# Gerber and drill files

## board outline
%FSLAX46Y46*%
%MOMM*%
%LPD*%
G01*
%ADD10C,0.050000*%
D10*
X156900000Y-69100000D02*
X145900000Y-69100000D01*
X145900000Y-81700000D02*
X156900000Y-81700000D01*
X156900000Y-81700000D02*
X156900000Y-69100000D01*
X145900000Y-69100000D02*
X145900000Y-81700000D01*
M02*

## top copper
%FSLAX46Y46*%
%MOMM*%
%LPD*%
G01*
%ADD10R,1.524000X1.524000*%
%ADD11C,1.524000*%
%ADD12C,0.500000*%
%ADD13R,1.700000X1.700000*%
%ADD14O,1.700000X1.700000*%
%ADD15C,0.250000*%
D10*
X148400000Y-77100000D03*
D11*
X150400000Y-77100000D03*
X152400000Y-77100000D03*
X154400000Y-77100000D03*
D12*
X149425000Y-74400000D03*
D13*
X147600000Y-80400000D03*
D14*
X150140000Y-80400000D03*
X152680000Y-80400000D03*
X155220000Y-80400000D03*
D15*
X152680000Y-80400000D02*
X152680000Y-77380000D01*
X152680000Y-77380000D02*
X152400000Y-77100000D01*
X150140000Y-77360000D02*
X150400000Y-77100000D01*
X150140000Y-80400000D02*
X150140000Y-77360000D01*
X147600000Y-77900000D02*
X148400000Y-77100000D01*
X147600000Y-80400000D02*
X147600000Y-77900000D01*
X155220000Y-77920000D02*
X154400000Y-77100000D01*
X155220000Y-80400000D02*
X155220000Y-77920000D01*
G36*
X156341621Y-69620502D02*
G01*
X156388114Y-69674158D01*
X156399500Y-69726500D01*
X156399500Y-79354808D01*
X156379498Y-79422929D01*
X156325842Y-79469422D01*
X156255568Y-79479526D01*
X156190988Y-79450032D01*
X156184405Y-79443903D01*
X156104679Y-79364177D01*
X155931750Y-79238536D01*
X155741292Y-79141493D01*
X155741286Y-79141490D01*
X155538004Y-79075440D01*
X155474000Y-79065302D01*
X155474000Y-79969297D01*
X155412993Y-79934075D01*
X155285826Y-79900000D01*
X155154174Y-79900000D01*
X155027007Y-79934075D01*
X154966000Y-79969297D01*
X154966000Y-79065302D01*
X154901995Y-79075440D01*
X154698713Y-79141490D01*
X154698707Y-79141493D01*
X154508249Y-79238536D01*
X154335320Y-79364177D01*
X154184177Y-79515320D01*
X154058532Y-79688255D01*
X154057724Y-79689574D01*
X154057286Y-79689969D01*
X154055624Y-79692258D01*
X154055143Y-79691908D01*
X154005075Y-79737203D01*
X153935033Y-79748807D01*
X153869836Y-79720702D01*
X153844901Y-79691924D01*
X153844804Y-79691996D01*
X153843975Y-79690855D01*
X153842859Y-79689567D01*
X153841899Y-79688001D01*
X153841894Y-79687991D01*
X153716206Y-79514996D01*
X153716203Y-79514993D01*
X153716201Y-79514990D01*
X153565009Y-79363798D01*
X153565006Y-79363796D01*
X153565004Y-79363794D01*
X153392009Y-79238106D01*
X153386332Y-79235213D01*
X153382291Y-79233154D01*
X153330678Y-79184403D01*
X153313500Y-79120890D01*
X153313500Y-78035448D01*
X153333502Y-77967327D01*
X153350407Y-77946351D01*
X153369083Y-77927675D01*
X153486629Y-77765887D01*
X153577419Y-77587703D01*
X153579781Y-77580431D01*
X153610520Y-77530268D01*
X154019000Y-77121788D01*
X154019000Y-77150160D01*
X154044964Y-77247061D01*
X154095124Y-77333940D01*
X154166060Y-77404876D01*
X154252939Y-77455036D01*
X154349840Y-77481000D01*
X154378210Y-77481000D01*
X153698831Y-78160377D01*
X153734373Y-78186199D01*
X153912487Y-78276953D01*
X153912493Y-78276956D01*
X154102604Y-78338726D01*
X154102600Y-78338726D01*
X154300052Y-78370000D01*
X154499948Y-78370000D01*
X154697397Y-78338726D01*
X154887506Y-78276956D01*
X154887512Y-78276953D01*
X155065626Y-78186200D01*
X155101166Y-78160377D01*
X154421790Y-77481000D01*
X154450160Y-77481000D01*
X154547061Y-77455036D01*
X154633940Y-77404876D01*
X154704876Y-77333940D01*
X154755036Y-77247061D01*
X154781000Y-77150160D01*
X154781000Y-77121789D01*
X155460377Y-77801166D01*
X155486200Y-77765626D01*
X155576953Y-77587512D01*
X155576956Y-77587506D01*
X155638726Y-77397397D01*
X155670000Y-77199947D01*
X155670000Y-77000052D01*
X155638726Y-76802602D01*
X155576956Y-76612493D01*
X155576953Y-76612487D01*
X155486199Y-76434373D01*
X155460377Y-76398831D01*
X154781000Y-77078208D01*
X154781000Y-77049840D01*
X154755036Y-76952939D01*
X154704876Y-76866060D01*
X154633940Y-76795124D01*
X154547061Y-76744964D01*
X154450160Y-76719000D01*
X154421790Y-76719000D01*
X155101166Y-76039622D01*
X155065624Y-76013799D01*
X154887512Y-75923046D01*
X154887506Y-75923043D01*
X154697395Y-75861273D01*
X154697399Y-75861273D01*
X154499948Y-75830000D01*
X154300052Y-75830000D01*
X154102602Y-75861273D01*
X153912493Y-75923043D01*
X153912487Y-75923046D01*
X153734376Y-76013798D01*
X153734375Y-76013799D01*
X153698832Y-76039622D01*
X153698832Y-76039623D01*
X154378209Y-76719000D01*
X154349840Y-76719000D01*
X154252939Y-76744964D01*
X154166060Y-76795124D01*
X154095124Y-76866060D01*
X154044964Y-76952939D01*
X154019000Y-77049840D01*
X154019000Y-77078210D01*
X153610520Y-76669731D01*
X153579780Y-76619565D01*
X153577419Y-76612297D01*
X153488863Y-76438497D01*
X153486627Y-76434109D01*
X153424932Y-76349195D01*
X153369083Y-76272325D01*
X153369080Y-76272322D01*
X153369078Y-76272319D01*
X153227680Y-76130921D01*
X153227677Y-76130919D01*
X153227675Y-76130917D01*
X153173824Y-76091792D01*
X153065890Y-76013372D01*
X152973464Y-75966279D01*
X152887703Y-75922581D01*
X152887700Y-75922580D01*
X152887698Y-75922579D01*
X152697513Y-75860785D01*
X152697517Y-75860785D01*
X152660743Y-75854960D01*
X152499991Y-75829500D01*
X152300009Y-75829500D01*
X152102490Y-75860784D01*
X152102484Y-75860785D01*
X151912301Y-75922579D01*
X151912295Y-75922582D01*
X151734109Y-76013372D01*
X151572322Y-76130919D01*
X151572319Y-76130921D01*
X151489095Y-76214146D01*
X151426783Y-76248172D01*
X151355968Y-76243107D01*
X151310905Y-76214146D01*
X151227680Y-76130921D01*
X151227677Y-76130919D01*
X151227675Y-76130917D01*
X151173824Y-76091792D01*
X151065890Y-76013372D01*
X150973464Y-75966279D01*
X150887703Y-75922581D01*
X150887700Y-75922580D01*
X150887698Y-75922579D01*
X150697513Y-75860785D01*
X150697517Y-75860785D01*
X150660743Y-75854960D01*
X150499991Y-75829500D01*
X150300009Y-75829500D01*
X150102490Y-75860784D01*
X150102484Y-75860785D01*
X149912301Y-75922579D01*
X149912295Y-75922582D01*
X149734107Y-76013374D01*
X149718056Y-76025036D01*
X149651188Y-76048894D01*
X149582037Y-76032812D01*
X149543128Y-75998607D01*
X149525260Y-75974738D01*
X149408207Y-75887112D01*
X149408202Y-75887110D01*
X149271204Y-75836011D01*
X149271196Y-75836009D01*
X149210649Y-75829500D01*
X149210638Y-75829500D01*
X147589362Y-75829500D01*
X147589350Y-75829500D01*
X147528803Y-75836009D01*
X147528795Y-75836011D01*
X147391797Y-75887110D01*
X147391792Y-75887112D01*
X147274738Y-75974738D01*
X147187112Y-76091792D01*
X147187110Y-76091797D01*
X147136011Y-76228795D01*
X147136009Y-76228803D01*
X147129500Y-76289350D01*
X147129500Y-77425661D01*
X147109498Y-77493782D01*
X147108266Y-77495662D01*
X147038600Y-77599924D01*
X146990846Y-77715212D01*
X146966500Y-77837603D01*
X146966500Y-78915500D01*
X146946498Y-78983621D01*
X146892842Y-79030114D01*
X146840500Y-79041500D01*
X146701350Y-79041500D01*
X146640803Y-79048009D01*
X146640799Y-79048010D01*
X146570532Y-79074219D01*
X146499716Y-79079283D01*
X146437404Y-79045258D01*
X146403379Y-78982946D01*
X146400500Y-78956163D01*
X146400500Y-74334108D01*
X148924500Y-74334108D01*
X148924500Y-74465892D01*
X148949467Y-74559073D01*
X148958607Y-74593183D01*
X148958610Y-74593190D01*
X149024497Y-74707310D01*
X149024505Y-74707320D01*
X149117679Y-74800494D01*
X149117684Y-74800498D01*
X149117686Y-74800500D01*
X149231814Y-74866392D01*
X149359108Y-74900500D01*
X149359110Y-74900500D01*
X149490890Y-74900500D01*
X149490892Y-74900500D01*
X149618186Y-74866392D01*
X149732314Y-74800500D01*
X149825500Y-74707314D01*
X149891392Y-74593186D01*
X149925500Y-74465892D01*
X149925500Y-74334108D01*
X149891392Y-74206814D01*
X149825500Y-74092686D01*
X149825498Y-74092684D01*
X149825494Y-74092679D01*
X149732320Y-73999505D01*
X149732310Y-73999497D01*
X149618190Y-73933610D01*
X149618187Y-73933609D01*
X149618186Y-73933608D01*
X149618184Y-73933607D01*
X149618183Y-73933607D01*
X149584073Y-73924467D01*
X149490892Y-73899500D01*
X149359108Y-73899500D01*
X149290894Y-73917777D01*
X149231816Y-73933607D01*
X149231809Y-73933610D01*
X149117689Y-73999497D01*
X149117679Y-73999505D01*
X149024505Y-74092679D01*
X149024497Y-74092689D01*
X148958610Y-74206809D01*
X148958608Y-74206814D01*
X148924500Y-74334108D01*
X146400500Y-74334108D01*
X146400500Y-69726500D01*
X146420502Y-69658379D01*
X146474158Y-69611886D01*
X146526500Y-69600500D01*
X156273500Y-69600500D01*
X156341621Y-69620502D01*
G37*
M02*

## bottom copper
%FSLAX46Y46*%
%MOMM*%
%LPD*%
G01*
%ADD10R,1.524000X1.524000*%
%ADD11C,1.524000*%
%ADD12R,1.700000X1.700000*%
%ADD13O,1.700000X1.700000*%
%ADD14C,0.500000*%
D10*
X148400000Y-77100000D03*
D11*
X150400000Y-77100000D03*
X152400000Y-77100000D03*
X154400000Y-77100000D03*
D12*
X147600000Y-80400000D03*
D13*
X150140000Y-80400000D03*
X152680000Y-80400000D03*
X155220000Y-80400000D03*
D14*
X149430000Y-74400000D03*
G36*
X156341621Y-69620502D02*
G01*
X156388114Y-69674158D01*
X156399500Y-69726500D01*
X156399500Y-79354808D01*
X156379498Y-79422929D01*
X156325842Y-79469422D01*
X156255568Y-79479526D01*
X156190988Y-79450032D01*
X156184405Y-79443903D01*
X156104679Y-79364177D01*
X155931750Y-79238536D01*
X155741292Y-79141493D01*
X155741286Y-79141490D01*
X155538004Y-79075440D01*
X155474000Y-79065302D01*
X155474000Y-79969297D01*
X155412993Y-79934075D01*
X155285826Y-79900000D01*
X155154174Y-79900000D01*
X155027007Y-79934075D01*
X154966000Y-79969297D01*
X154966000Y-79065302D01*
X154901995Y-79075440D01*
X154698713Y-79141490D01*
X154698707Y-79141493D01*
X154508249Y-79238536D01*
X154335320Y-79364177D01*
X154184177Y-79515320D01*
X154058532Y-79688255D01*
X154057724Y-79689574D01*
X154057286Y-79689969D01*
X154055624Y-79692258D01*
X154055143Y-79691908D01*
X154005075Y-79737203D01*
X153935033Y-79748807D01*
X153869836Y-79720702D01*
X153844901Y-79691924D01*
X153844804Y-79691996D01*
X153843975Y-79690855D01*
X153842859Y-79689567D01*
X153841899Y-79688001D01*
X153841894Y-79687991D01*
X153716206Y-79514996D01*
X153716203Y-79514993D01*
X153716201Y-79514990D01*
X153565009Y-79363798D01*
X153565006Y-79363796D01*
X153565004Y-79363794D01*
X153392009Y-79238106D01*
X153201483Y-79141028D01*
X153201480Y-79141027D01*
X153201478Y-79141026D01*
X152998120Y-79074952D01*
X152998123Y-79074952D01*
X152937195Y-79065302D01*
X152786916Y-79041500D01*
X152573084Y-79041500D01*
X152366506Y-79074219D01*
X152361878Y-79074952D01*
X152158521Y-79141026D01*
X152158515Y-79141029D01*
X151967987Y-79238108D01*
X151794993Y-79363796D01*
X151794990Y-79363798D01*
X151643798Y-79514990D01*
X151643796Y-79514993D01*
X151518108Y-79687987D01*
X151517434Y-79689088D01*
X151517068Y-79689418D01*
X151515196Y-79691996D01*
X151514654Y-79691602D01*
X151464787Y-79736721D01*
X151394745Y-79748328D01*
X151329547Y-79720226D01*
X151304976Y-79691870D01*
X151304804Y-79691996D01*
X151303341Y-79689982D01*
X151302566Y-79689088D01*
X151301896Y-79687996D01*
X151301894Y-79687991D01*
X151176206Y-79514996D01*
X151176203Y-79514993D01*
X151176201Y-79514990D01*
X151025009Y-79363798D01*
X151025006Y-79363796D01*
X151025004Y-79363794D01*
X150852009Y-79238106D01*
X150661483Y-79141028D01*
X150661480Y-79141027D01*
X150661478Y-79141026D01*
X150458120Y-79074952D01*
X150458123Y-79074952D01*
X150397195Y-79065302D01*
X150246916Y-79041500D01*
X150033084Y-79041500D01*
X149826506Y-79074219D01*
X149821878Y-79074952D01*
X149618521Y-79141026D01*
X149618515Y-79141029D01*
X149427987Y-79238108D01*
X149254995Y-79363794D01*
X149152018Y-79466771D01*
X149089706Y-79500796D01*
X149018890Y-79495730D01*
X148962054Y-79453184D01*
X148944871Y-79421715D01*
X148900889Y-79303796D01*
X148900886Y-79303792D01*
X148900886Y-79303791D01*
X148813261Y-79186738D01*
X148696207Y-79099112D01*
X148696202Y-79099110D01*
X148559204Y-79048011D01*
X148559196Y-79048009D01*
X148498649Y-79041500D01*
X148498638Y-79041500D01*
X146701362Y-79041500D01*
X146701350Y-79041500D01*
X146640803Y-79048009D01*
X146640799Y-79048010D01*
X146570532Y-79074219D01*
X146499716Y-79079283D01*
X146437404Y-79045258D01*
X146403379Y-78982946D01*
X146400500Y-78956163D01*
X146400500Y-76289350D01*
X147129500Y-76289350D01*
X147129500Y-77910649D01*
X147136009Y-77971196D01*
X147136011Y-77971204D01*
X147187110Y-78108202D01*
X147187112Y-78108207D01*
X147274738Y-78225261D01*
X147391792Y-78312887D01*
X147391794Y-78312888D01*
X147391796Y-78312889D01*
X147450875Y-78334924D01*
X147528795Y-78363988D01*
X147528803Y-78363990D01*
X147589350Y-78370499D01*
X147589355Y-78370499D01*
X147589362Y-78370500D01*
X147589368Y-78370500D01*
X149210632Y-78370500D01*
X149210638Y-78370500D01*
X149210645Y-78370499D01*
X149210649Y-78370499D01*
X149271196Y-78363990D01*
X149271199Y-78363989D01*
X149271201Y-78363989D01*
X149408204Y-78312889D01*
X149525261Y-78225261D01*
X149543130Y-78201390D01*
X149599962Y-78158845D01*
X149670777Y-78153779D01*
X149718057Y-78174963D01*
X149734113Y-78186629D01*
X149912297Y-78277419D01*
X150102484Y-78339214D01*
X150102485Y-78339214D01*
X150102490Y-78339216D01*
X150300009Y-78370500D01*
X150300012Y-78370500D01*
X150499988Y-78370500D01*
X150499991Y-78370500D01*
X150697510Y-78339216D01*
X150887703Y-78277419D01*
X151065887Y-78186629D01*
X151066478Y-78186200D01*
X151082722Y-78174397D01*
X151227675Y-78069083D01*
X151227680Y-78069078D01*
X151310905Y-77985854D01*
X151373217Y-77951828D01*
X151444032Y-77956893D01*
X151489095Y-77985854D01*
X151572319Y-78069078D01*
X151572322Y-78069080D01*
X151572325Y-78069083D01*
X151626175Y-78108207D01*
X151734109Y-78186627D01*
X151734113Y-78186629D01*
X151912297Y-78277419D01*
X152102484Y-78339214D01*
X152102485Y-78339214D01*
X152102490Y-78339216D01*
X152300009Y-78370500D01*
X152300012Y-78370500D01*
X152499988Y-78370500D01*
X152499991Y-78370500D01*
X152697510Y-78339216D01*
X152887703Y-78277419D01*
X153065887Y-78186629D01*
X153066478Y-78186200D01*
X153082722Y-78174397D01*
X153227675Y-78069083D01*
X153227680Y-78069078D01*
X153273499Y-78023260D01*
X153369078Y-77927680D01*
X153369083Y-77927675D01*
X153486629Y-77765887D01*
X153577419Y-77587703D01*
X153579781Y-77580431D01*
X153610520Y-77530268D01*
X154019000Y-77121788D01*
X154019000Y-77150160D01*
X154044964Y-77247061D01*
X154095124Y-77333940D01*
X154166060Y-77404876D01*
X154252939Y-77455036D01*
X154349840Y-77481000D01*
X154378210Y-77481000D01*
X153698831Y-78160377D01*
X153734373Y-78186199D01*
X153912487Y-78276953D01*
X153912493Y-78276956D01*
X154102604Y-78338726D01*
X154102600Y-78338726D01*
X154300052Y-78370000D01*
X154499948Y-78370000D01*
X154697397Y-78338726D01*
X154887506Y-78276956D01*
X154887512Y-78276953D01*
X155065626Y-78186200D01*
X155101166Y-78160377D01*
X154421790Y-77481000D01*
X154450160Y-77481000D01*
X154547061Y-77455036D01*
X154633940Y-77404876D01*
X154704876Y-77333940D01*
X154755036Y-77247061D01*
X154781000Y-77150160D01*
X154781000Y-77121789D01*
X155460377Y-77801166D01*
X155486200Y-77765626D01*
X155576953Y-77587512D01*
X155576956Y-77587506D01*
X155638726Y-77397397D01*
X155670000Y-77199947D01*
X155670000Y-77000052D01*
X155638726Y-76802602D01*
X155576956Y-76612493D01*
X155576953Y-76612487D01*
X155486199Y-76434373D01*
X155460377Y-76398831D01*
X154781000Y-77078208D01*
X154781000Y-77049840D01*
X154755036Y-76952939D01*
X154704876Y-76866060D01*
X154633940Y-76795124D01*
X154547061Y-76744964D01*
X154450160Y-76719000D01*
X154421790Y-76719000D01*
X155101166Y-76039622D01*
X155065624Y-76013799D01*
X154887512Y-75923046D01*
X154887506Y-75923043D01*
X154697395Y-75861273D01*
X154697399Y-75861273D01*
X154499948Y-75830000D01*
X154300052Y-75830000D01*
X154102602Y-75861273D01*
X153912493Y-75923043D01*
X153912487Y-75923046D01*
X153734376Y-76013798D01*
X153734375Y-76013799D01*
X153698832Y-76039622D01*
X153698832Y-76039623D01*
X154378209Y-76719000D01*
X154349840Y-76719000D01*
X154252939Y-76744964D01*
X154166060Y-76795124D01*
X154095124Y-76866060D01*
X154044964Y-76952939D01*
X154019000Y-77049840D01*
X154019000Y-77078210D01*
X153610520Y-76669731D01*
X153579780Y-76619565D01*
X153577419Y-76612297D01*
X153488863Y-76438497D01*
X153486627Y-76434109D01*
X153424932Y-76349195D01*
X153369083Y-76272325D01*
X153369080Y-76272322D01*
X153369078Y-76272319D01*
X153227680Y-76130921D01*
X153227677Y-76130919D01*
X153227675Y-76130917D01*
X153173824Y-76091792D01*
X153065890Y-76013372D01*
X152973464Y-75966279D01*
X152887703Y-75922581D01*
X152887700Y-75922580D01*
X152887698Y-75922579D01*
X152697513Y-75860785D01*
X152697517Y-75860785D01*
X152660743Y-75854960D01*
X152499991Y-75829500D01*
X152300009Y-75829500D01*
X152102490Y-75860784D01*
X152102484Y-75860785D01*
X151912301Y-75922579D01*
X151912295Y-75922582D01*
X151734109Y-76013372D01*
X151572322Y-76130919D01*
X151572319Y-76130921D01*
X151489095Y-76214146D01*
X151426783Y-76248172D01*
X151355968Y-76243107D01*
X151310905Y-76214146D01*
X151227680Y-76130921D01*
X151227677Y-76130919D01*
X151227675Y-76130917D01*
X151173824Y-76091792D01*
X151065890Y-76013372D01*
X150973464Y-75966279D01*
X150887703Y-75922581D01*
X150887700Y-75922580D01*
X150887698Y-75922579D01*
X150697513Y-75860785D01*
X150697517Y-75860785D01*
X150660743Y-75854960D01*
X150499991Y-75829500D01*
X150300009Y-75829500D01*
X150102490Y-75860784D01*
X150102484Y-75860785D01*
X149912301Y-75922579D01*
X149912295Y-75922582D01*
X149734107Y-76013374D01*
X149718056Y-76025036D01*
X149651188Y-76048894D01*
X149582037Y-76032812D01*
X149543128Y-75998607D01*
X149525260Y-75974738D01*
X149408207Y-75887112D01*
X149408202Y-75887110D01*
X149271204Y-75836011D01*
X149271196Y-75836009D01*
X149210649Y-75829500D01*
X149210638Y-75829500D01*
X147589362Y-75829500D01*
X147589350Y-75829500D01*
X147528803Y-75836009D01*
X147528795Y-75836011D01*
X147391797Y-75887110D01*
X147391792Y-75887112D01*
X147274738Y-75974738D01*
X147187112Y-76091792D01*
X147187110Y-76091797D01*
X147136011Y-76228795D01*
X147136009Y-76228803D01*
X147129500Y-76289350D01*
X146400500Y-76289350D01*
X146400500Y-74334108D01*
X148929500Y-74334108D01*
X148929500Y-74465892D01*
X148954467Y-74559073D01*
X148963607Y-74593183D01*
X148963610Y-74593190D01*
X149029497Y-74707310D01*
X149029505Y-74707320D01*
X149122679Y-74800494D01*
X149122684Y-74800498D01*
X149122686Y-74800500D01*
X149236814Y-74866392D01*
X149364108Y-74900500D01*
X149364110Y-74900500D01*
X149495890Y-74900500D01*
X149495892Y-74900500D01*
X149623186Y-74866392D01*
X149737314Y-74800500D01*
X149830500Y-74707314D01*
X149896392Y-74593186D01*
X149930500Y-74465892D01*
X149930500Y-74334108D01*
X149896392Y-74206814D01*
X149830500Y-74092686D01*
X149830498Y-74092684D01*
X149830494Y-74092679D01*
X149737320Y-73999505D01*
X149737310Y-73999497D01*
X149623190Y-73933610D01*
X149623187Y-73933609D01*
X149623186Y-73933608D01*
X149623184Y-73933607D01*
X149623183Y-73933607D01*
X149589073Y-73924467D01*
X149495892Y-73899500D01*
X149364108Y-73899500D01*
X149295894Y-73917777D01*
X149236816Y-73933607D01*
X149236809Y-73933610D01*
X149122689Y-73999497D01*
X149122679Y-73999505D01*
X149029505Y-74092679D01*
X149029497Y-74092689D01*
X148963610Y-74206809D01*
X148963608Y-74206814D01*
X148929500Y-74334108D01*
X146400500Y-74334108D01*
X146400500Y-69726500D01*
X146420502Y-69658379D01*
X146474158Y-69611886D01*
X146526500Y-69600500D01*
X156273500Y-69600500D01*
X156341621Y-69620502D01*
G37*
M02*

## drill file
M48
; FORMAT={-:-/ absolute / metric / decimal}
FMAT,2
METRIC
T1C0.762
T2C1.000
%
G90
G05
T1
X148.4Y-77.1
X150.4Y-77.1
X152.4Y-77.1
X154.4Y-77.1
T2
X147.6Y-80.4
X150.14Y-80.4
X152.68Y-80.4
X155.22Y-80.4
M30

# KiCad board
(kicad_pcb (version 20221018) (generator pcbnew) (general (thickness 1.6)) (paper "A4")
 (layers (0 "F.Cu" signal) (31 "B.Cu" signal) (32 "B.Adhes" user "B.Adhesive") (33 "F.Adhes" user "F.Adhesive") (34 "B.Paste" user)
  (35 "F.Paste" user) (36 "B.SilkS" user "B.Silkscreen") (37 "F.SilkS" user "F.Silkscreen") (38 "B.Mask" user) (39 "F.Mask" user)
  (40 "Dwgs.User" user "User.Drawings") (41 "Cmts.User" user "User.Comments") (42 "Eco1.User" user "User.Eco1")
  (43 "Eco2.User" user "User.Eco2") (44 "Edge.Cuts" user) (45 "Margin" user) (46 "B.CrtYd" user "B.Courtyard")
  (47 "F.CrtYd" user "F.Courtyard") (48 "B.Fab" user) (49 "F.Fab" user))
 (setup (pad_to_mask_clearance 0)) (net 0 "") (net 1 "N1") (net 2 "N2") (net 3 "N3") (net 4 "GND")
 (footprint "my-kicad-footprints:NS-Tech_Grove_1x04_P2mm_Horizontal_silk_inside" (layer "F.Cu") (at 151.4 77.1 90)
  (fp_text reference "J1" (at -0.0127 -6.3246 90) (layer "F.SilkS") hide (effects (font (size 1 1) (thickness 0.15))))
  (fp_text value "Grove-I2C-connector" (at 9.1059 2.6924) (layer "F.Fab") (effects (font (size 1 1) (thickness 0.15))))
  (pad "1" thru_hole rect (at 0 -3 90) (size 1.524 1.524) (drill 0.762) (layers "*.Cu" "*.Mask") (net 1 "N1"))
  (pad "2" thru_hole circle (at 0 -1 90) (size 1.524 1.524) (drill 0.762) (layers "*.Cu" "*.Mask") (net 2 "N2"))
  (pad "3" thru_hole circle (at 0 1 90) (size 1.524 1.524) (drill 0.762) (layers "*.Cu" "*.Mask") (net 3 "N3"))
  (pad "4" thru_hole circle (at 0 3 90) (size 1.524 1.524) (drill 0.762) (layers "*.Cu" "*.Mask") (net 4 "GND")))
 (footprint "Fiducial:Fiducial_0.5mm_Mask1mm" (layer "F.Cu") (at 149.425 74.4)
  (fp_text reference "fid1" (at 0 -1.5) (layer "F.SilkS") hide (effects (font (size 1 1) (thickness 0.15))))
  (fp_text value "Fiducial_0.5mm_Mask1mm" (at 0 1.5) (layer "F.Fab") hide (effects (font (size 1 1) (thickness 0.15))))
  (pad "" smd circle (at 0 0) (size 0.5 0.5) (layers "F.Cu" "F.Mask") (solder_mask_margin 0.25) (clearance 0.25)))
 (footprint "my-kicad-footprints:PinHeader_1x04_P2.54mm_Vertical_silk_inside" (layer "B.Cu") (at 147.6 80.4 -90)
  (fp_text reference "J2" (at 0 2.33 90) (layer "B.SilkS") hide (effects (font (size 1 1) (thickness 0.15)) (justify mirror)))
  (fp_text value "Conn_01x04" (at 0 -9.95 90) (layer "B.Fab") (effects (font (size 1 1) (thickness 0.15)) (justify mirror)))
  (pad "1" thru_hole rect (at 0 0 270) (size 1.7 1.7) (drill 1) (layers "*.Cu" "*.Mask") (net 1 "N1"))
  (pad "2" thru_hole oval (at 0 -2.54 270) (size 1.7 1.7) (drill 1) (layers "*.Cu" "*.Mask") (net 2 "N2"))
  (pad "3" thru_hole oval (at 0 -5.08 270) (size 1.7 1.7) (drill 1) (layers "*.Cu" "*.Mask") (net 3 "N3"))
  (pad "4" thru_hole oval (at 0 -7.62 270) (size 1.7 1.7) (drill 1) (layers "*.Cu" "*.Mask") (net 4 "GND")))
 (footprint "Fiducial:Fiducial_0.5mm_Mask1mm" (layer "B.Cu") (at 149.43 74.4)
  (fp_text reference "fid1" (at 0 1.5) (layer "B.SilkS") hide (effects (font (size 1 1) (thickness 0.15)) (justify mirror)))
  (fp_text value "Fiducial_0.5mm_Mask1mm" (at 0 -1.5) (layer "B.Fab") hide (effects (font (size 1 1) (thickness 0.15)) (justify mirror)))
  (pad "" smd circle (at 0 0) (size 0.5 0.5) (layers "B.Cu" "B.Mask") (solder_mask_margin 0.25) (clearance 0.25)))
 (gr_line (start 156.9 69.1) (end 145.9 69.1) (stroke (width 0.05) (type solid)) (layer "Edge.Cuts"))
 (gr_line (start 145.9 81.7) (end 156.9 81.7) (stroke (width 0.05) (type solid)) (layer "Edge.Cuts"))
 (gr_line (start 156.9 81.7) (end 156.9 69.1) (stroke (width 0.05) (type solid)) (layer "Edge.Cuts"))
 (gr_line (start 145.9 69.1) (end 145.9 81.7) (stroke (width 0.05) (type solid)) (layer "Edge.Cuts"))
 (segment (start 152.68 80.4) (end 152.68 77.38) (width 0.25) (layer "F.Cu") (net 3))
 (segment (start 152.68 77.38) (end 152.4 77.1) (width 0.25) (layer "F.Cu") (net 3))
 (segment (start 150.14 77.36) (end 150.4 77.1) (width 0.25) (layer "F.Cu") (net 2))
 (segment (start 150.14 80.4) (end 150.14 77.36) (width 0.25) (layer "F.Cu") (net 2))
 (segment (start 147.6 77.9) (end 148.4 77.1) (width 0.25) (layer "F.Cu") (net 1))
 (segment (start 147.6 80.4) (end 147.6 77.9) (width 0.25) (layer "F.Cu") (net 1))
 (segment (start 155.22 77.92) (end 154.4 77.1) (width 0.25) (layer "F.Cu") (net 4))
 (segment (start 155.22 80.4) (end 155.22 77.92) (width 0.25) (layer "F.Cu") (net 4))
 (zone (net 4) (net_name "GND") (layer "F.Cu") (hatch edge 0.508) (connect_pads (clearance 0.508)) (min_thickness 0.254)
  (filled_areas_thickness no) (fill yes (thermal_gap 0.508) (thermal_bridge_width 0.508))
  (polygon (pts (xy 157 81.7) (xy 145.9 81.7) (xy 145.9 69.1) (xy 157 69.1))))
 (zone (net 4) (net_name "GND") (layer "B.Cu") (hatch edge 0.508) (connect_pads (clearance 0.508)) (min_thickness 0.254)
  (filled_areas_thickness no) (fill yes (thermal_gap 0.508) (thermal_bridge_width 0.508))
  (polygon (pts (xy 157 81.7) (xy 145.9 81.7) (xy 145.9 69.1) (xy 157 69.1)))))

